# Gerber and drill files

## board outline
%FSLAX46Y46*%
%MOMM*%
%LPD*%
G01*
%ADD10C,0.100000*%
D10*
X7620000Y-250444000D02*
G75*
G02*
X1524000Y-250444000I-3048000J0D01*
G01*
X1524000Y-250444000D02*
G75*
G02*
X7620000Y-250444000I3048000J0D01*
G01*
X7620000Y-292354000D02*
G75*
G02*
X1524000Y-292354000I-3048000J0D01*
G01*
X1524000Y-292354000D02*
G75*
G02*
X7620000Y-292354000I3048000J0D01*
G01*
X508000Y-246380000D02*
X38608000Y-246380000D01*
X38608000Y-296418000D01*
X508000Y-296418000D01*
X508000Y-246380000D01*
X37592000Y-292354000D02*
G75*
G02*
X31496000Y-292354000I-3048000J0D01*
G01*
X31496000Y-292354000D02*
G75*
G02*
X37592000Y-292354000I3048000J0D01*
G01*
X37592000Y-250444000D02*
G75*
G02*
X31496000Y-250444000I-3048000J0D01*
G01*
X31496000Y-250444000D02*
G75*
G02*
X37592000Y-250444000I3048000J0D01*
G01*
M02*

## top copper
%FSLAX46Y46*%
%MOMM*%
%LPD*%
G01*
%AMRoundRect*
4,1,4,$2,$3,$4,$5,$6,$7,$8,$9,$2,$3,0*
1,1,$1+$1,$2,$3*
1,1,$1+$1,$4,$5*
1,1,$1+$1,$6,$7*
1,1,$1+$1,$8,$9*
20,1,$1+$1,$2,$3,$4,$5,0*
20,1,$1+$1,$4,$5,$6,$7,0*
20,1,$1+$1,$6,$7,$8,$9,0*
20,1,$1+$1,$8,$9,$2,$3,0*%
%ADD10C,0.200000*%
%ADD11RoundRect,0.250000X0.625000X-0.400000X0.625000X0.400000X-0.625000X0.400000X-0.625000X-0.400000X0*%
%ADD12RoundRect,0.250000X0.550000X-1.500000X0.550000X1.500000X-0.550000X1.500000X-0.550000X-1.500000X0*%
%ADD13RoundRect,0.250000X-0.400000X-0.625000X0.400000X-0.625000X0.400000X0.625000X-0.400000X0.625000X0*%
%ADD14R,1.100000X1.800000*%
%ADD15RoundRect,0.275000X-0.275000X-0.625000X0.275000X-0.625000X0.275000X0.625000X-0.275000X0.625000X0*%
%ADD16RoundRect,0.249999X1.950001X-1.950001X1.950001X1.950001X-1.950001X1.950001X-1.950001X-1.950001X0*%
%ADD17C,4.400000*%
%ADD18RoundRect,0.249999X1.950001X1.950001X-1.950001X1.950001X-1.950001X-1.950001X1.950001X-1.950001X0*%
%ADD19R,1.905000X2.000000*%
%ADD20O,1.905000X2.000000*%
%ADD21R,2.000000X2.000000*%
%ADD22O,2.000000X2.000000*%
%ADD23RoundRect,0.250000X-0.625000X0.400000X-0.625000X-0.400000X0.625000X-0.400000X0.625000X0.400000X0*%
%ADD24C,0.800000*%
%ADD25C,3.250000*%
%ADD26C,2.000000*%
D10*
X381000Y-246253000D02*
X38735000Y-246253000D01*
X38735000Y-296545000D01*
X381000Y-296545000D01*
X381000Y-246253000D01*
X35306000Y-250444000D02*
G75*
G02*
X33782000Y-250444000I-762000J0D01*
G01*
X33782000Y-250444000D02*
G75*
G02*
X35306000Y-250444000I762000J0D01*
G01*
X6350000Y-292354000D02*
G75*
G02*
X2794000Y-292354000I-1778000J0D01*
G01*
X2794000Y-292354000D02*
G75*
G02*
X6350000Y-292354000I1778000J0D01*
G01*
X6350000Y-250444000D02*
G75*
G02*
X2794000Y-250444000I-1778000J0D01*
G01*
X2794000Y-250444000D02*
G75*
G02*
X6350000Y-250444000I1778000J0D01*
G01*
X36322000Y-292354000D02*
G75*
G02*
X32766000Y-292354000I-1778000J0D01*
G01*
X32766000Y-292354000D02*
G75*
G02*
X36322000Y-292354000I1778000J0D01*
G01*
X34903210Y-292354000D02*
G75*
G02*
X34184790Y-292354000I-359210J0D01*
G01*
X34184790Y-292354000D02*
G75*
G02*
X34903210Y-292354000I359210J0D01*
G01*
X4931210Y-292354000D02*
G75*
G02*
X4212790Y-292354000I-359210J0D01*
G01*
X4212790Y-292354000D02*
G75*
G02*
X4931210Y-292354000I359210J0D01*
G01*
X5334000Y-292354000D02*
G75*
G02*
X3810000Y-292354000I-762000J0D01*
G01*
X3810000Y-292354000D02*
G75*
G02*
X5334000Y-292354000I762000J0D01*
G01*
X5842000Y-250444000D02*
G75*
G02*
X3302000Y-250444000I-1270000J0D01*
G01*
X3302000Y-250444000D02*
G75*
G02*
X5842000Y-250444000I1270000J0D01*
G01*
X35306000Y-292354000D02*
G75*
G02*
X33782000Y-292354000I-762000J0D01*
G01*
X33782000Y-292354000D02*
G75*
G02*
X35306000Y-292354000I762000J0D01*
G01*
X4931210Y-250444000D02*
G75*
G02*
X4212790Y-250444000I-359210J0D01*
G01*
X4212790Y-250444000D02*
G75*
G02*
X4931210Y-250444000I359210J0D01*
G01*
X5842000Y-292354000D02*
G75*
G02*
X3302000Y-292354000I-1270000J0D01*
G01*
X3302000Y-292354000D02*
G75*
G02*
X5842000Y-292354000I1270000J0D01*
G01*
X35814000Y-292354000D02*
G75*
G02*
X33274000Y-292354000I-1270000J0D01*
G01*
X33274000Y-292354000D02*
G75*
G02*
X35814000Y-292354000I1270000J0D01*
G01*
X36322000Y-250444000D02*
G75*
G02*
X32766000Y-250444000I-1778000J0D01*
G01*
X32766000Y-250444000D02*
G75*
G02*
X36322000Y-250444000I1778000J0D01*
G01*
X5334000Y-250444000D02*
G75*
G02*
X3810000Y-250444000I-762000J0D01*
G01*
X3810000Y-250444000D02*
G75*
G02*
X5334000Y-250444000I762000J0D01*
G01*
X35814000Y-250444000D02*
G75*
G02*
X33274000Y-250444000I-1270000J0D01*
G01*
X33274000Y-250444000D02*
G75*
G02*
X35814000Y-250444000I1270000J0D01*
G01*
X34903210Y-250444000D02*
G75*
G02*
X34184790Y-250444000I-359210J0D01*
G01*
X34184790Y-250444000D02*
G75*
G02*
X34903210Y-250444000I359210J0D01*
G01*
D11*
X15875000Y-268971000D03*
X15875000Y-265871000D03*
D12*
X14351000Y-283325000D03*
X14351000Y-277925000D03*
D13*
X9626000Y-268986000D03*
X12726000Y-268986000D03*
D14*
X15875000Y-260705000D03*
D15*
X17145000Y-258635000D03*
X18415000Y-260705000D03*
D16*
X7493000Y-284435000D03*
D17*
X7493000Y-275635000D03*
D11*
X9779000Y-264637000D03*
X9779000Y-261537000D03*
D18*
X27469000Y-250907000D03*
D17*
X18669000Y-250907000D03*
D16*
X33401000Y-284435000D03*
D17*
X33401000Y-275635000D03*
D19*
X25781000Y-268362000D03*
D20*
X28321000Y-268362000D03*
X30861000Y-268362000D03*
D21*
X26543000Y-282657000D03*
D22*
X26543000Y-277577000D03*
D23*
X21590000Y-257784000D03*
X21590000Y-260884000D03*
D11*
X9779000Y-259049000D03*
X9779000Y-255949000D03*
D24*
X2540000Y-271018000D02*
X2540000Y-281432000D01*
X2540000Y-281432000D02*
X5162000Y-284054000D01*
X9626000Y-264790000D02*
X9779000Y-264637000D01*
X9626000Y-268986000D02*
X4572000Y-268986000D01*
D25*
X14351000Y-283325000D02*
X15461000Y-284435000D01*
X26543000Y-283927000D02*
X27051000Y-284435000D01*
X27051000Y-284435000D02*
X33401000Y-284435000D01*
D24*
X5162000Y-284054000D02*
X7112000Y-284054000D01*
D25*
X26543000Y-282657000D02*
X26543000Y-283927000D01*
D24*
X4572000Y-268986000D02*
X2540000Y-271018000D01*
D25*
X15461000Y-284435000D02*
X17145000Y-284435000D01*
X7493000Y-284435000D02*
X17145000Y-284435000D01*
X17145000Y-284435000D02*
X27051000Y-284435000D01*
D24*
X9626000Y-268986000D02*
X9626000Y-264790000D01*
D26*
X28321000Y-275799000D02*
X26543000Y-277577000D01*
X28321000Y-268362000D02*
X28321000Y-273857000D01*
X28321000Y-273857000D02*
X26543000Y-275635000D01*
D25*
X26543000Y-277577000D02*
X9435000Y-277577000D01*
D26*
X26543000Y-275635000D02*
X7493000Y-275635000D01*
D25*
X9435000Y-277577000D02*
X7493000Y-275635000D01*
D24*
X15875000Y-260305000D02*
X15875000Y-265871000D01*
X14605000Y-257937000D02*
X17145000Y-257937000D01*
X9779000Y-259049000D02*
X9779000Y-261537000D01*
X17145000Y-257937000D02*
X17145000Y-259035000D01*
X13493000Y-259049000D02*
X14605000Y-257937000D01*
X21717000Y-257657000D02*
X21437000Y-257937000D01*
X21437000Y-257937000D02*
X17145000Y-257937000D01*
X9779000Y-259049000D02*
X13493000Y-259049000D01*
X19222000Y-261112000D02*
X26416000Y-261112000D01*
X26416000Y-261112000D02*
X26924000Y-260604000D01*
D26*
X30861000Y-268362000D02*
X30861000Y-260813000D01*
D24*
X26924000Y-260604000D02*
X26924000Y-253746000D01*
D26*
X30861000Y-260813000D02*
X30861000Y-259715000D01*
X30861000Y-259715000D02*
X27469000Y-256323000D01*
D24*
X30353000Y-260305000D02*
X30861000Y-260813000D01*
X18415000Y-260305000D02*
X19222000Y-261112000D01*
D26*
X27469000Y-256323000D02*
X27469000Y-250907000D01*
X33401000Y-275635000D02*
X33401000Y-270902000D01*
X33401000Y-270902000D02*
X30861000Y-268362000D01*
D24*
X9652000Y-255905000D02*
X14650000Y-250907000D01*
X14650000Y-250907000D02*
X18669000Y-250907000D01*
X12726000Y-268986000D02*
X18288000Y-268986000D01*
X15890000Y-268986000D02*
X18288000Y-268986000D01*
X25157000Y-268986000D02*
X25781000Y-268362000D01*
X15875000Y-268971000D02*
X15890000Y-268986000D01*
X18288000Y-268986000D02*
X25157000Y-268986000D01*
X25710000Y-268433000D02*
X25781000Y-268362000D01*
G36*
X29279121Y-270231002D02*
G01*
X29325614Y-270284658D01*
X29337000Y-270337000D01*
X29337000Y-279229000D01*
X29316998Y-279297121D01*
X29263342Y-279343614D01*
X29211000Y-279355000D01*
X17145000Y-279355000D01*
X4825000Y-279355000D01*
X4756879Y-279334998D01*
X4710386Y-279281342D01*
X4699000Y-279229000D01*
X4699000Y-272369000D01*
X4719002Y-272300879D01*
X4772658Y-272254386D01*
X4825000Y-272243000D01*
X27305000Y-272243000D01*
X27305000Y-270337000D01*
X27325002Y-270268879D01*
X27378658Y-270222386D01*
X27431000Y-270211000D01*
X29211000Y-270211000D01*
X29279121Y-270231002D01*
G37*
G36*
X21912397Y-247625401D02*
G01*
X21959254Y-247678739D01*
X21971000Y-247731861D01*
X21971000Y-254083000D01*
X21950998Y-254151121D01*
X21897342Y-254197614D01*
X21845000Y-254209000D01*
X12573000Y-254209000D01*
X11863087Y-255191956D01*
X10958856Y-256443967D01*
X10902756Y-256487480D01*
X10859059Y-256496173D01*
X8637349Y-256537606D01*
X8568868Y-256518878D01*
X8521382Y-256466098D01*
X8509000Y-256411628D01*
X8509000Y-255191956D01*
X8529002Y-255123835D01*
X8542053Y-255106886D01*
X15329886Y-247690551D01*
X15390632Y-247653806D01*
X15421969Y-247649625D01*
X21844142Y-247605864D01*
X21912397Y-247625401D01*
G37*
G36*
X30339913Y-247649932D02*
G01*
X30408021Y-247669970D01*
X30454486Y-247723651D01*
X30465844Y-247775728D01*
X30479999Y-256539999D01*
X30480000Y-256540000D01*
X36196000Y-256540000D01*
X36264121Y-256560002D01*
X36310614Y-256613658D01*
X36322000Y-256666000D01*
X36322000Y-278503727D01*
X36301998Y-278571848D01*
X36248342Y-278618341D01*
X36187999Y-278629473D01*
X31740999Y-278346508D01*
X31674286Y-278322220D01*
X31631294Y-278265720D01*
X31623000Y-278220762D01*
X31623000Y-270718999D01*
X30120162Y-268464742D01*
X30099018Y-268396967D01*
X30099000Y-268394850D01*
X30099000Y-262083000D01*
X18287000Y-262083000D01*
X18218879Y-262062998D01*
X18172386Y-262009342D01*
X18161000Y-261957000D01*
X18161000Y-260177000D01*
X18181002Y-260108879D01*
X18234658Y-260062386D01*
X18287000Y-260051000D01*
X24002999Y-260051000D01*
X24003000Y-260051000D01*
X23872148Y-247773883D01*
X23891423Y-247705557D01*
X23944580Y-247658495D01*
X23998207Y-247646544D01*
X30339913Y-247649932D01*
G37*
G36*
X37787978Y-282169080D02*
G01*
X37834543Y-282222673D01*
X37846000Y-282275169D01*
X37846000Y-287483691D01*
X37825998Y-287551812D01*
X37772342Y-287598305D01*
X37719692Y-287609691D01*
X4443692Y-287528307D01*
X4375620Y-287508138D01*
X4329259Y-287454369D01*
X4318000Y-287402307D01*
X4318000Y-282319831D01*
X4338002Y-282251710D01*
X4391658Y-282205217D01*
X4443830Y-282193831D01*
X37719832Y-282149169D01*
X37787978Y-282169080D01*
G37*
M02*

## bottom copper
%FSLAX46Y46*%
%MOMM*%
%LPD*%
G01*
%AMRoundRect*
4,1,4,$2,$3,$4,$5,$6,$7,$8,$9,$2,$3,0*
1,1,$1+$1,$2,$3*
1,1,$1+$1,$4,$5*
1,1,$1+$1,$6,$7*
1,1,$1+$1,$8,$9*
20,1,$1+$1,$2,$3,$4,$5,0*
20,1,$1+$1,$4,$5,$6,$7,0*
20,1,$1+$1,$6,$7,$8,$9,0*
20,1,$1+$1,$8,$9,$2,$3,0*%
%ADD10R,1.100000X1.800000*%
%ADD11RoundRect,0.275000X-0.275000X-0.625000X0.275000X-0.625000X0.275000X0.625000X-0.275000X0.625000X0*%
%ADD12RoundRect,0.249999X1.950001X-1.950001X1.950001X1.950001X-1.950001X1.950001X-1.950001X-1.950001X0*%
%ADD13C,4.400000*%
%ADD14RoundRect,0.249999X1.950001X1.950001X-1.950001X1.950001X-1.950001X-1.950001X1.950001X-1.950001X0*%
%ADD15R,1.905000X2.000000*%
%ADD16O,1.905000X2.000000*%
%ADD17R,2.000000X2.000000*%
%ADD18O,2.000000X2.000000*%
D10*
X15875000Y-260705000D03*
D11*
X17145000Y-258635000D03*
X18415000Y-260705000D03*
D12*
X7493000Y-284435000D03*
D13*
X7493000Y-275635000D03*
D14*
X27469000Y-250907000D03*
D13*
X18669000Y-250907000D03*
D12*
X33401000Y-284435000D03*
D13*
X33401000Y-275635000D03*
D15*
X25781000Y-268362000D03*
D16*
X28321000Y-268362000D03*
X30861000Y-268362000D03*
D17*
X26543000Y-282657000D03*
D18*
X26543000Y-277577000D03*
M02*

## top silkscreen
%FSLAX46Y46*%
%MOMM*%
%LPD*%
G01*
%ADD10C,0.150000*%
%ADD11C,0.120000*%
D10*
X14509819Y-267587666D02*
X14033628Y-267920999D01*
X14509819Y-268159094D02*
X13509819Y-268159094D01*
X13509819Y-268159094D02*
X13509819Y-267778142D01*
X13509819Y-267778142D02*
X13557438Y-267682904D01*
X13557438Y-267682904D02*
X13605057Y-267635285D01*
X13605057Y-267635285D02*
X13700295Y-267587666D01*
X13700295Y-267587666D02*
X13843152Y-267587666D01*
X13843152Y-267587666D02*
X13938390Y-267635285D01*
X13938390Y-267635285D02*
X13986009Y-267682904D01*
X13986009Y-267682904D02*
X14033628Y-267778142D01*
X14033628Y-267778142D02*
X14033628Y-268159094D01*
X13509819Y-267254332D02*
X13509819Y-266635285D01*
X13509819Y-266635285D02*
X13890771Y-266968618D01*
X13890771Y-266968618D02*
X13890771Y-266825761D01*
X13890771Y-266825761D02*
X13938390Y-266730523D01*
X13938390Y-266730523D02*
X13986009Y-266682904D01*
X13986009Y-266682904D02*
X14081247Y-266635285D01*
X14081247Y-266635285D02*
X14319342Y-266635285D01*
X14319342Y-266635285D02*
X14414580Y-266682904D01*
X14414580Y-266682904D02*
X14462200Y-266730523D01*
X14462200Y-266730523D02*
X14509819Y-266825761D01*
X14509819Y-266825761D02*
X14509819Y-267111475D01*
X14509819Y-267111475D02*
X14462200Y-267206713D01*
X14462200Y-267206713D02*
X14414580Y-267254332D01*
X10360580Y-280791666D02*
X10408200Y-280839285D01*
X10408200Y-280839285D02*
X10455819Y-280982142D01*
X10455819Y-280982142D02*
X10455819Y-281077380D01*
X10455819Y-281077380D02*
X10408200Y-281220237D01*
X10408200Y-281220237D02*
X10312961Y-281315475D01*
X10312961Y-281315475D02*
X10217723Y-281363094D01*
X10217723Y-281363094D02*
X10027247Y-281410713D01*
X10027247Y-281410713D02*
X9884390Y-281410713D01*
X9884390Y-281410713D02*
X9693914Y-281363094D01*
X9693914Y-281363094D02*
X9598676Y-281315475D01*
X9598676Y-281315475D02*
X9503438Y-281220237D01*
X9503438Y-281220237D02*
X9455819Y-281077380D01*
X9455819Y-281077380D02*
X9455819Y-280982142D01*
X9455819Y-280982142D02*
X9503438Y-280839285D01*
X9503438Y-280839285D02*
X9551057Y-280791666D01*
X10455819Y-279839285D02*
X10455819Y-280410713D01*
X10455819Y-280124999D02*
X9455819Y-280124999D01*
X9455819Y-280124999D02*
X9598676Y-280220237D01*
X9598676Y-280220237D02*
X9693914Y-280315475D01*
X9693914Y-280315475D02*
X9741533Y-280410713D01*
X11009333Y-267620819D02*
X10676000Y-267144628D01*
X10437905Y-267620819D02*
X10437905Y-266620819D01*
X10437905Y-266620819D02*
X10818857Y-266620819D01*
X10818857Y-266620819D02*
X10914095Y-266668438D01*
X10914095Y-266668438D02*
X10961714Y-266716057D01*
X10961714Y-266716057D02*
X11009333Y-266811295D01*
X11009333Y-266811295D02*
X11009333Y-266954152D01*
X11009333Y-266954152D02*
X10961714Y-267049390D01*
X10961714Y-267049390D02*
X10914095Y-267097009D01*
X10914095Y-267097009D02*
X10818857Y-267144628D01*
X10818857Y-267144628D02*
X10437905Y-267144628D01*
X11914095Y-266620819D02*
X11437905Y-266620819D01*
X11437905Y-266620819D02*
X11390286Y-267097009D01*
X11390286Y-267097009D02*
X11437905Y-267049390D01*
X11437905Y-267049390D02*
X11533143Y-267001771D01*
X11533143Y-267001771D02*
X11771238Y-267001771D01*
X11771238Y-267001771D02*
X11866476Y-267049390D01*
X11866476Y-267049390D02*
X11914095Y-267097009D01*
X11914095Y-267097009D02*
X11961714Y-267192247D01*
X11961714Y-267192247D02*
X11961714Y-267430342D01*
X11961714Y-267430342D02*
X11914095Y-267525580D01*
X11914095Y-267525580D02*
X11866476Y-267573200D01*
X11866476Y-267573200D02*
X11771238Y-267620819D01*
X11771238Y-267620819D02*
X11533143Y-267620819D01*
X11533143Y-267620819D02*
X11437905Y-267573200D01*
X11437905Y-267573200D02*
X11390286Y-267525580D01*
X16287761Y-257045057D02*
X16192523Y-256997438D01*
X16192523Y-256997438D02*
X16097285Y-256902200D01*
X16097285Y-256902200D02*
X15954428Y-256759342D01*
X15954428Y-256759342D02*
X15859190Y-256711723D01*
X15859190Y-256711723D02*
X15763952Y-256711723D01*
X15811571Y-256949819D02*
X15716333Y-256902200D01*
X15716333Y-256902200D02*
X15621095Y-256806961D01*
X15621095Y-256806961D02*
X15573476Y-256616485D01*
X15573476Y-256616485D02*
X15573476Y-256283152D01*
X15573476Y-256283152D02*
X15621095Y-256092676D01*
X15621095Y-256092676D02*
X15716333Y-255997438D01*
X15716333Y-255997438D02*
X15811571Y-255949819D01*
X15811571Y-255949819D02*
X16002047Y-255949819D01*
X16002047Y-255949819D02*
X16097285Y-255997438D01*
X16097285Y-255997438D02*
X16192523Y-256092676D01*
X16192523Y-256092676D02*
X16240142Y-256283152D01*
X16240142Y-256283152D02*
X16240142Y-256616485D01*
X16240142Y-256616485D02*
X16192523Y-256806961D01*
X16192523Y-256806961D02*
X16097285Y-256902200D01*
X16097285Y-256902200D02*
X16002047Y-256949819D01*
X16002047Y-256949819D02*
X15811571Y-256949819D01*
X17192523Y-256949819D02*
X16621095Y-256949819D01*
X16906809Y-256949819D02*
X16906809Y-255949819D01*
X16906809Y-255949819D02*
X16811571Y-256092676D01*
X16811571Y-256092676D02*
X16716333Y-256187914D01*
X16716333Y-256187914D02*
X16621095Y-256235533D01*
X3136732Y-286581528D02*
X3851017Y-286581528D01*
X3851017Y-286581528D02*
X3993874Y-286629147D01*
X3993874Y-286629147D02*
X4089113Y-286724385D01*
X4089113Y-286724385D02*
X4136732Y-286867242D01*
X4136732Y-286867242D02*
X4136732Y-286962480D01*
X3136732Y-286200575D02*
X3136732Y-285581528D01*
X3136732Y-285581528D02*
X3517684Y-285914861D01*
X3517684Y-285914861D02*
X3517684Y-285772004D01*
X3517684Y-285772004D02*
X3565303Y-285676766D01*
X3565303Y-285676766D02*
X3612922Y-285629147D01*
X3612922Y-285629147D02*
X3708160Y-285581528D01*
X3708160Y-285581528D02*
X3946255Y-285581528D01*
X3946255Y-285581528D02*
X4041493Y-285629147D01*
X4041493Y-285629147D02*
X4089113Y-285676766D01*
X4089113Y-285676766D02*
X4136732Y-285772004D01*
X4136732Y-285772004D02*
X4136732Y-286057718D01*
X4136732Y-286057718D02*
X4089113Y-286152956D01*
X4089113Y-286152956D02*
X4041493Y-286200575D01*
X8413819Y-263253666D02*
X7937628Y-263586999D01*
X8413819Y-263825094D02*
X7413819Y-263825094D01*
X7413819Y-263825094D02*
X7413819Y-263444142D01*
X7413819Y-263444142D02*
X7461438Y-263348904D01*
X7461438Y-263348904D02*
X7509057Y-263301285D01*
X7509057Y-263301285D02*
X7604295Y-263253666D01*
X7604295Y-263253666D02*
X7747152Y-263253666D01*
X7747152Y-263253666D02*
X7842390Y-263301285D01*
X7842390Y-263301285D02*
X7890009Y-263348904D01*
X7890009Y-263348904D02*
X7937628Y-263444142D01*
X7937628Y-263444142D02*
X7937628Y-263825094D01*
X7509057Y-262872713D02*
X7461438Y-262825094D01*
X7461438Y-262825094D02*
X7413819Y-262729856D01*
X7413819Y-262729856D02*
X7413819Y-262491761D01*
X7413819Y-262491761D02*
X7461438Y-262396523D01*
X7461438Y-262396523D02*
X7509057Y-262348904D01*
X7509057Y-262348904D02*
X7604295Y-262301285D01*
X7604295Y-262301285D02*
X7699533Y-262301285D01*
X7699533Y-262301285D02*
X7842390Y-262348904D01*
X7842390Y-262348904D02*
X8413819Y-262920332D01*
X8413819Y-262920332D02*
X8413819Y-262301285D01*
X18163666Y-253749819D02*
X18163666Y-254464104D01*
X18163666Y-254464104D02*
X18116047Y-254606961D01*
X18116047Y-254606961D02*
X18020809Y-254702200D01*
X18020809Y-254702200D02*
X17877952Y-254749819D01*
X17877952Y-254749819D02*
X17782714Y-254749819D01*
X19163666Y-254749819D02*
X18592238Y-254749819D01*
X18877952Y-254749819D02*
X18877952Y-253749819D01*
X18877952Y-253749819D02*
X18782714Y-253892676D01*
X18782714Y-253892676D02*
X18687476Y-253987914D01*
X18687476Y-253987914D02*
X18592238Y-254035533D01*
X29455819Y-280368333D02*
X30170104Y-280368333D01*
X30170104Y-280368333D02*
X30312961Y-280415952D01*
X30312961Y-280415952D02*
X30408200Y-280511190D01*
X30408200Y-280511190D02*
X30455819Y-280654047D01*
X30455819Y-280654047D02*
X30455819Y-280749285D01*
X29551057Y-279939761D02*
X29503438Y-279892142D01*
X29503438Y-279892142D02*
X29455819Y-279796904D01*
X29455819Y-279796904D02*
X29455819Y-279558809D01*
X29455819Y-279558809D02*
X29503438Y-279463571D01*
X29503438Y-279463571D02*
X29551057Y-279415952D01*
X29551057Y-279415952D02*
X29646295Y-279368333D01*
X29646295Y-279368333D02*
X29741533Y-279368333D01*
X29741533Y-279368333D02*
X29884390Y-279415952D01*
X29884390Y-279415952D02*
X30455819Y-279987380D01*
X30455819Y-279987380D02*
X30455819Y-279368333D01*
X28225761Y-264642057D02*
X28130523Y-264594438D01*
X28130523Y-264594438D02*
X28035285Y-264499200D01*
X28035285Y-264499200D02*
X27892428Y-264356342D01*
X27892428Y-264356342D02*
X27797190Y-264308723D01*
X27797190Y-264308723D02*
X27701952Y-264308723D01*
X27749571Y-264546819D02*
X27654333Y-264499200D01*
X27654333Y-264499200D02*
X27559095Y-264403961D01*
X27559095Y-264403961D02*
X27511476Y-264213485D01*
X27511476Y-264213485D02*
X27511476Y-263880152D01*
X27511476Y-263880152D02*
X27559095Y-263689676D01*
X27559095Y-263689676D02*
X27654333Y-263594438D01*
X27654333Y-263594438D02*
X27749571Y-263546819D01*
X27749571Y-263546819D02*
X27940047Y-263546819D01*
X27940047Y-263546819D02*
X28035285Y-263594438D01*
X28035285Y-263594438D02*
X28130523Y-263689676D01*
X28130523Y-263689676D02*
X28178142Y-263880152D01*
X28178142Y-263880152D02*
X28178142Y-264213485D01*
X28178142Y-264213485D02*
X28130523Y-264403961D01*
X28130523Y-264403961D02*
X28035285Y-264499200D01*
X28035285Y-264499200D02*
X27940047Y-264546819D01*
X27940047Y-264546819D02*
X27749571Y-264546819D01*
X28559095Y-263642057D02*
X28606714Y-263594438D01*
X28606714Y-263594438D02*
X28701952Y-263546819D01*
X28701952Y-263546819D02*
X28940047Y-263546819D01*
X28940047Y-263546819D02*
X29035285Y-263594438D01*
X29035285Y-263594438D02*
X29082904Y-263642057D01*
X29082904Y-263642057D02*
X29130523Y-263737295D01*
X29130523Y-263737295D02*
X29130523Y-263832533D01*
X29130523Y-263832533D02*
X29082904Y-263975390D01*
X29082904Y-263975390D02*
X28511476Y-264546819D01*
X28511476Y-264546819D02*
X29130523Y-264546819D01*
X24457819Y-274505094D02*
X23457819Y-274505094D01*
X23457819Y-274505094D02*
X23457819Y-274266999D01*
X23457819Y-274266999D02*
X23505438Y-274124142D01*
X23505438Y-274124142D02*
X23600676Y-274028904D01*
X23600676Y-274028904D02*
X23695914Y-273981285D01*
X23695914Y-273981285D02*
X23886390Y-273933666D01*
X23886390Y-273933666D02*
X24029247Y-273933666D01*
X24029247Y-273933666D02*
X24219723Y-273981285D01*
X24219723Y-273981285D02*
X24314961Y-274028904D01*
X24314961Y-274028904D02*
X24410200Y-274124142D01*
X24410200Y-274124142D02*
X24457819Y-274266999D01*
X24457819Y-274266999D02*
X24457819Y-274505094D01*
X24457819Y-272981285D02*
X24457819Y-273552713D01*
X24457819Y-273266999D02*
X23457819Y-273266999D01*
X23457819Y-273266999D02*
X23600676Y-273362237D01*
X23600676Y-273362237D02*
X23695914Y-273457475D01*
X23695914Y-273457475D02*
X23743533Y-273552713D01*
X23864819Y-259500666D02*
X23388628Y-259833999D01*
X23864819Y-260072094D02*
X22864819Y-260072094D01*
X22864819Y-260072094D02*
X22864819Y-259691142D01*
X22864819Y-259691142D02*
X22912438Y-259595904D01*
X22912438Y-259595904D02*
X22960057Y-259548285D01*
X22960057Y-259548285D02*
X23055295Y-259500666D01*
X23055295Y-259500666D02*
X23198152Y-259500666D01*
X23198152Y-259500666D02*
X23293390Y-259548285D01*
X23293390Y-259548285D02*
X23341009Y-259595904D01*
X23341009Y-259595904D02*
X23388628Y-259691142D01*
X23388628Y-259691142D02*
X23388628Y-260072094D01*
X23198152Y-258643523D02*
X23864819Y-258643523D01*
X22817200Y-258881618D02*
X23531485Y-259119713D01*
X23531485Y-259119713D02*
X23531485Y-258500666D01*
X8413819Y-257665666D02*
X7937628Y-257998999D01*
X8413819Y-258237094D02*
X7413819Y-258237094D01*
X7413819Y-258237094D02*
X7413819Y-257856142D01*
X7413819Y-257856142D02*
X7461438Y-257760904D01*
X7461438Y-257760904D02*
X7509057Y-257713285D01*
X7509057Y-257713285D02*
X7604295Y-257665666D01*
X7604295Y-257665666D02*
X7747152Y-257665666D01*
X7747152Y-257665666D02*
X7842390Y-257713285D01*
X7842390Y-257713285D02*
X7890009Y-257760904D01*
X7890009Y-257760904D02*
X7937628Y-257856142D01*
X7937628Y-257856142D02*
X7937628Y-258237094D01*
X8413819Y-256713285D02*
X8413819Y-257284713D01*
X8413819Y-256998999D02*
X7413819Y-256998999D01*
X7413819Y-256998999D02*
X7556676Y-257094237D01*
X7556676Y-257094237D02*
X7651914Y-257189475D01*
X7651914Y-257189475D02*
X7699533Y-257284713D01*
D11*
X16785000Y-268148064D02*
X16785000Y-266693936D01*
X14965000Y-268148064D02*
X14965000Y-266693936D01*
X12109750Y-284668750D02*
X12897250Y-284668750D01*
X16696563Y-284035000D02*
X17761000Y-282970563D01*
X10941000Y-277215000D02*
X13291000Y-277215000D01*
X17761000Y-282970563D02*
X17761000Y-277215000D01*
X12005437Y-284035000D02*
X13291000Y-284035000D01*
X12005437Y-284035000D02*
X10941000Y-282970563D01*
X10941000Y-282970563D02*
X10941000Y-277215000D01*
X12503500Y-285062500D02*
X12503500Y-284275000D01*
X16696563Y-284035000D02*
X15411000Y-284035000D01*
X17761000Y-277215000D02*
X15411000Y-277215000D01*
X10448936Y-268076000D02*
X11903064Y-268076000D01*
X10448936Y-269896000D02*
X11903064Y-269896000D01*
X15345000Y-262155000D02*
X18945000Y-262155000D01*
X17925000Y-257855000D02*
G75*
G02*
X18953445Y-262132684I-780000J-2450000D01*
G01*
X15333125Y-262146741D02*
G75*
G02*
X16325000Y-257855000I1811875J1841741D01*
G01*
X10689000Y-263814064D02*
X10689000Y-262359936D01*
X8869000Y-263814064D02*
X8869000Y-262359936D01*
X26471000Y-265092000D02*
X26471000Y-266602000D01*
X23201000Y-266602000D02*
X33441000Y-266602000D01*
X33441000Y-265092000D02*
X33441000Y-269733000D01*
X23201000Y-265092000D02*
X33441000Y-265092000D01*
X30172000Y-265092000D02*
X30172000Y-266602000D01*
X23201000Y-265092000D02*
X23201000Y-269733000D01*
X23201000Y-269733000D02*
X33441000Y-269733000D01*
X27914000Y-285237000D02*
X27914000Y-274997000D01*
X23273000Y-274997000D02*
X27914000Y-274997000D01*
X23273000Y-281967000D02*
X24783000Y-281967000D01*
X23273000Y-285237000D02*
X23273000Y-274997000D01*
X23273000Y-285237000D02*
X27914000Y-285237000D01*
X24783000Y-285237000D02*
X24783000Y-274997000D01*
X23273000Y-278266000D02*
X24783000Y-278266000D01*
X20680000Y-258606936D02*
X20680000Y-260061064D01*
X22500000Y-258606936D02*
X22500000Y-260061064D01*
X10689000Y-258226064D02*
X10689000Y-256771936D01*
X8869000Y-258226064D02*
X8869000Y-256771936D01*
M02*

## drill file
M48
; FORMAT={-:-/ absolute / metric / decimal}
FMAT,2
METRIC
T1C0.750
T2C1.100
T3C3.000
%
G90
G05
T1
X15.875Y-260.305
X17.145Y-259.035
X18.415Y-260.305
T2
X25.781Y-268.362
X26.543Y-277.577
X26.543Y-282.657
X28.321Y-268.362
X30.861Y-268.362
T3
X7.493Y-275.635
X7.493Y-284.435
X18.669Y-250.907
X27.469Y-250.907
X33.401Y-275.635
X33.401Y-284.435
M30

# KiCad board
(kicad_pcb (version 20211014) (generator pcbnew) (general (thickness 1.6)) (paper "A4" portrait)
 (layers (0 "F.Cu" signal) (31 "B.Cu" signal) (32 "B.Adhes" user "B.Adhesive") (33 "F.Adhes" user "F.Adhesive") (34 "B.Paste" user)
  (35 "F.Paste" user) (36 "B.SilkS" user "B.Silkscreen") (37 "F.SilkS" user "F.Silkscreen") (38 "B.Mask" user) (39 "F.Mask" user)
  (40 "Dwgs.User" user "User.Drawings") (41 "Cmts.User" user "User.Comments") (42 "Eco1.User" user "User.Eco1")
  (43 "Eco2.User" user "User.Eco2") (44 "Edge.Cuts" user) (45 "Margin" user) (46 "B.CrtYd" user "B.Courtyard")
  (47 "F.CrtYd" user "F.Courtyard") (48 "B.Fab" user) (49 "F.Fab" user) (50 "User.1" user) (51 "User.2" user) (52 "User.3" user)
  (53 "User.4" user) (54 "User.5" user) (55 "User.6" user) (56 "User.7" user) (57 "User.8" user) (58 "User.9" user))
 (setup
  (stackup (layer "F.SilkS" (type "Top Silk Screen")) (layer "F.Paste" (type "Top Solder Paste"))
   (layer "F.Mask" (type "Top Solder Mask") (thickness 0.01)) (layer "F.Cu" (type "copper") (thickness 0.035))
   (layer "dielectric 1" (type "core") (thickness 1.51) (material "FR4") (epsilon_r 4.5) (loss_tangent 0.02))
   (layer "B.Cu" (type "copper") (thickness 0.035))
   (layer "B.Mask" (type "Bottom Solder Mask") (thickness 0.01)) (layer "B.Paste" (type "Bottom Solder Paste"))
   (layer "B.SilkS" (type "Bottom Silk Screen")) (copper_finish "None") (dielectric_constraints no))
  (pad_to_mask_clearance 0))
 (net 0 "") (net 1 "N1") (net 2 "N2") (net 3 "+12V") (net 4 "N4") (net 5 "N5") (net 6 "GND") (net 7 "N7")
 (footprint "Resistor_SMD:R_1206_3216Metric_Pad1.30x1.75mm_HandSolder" (layer "F.Cu") (at 15.875 267.421 90)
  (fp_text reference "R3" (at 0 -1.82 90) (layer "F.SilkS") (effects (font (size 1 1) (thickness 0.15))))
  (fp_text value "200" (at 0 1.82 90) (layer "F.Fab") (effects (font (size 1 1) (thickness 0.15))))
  (fp_line (start -0.727064 0.91) (end 0.727064 0.91) (layer "F.SilkS") (width 0.12))
  (fp_line (start -0.727064 -0.91) (end 0.727064 -0.91) (layer "F.SilkS") (width 0.12))
  (pad "1" smd roundrect (at -1.55 0 90) (size 1.3 1.75) (layers "F.Cu" "F.Paste" "F.Mask") (roundrect_rratio 0.192308) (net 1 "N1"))
  (pad "2" smd roundrect (at 1.55 0 90) (size 1.3 1.75) (layers "F.Cu" "F.Paste" "F.Mask") (roundrect_rratio 0.192308) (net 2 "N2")))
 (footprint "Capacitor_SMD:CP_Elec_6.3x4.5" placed (layer "F.Cu") (at 14.351 280.625 90)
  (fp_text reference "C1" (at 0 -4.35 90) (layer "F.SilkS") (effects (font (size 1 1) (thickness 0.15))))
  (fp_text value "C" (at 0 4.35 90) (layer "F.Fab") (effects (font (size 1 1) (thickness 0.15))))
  (fp_line (start -4.04375 -2.24125) (end -4.04375 -1.45375) (layer "F.SilkS") (width 0.12))
  (fp_line (start -3.41 2.345563) (end -2.345563 3.41) (layer "F.SilkS") (width 0.12))
  (fp_line (start 3.41 -3.41) (end 3.41 -1.06) (layer "F.SilkS") (width 0.12))
  (fp_line (start -2.345563 3.41) (end 3.41 3.41) (layer "F.SilkS") (width 0.12))
  (fp_line (start -3.41 -2.345563) (end -3.41 -1.06) (layer "F.SilkS") (width 0.12))
  (fp_line (start -3.41 -2.345563) (end -2.345563 -3.41) (layer "F.SilkS") (width 0.12))
  (fp_line (start -2.345563 -3.41) (end 3.41 -3.41) (layer "F.SilkS") (width 0.12))
  (fp_line (start -4.4375 -1.8475) (end -3.65 -1.8475) (layer "F.SilkS") (width 0.12))
  (fp_line (start -3.41 2.345563) (end -3.41 1.06) (layer "F.SilkS") (width 0.12))
  (fp_line (start 3.41 3.41) (end 3.41 1.06) (layer "F.SilkS") (width 0.12))
  (pad "1" smd roundrect (at -2.7 0 90) (size 3.5 1.6) (layers "F.Cu" "F.Paste" "F.Mask") (roundrect_rratio 0.15625) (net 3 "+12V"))
  (pad "2" smd roundrect (at 2.7 0 90) (size 3.5 1.6) (layers "F.Cu" "F.Paste" "F.Mask") (roundrect_rratio 0.15625) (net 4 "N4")))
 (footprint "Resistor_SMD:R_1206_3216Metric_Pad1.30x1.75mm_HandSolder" (layer "F.Cu") (at 11.176 268.986)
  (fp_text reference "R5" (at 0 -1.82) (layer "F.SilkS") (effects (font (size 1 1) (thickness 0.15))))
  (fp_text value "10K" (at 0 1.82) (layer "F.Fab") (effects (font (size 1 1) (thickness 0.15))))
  (fp_line (start -0.727064 -0.91) (end 0.727064 -0.91) (layer "F.SilkS") (width 0.12))
  (fp_line (start -0.727064 0.91) (end 0.727064 0.91) (layer "F.SilkS") (width 0.12))
  (pad "1" smd roundrect (at -1.55 0) (size 1.3 1.75) (layers "F.Cu" "F.Paste" "F.Mask") (roundrect_rratio 0.192308) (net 3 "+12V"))
  (pad "2" smd roundrect (at 1.55 0) (size 1.3 1.75) (layers "F.Cu" "F.Paste" "F.Mask") (roundrect_rratio 0.192308) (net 1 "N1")))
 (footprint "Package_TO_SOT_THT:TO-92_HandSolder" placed (layer "F.Cu") (at 15.875 260.305)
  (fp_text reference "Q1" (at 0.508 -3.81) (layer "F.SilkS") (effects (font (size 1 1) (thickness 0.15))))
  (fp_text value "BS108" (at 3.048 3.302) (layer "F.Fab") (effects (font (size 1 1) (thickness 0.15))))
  (fp_line (start -0.53 1.85) (end 3.07 1.85) (layer "F.SilkS") (width 0.12))
  (fp_arc (start 2.05 -2.45) (mid 3.769931 -0.601036) (end 3.078445 1.827684) (layer "F.SilkS") (width 0.12))
  (fp_arc (start -0.541875 1.841741) (mid -1.247231 -0.581764) (end 0.45 -2.45) (layer "F.SilkS") (width 0.12))
  (pad "1" thru_hole rect (at 0 0) (size 1.1 1.8) (drill 0.75 (offset 0 0.4)) (layers *.Cu *.Mask) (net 2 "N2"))
  (pad "2" thru_hole roundrect (at 1.27 -1.27) (size 1.1 1.8) (drill 0.75 (offset 0 -0.4)) (layers *.Cu *.Mask) (roundrect_rratio 0.25)
   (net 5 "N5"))
  (pad "3" thru_hole roundrect (at 2.54 0) (size 1.1 1.8) (drill 0.75 (offset 0 0.4)) (layers *.Cu *.Mask) (roundrect_rratio 0.25)
   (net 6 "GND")))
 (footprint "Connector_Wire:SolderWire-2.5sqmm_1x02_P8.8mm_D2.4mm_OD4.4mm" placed (layer "F.Cu") (at 7.493 284.435 90)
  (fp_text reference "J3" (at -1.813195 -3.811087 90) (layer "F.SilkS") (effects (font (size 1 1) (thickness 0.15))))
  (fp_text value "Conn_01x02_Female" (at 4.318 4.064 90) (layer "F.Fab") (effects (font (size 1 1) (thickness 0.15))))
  (pad "1" thru_hole roundrect (at 0 0 90) (size 4.4 4.4) (drill 3) (layers *.Cu *.Mask) (roundrect_rratio 0.05681795455) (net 3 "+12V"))
  (pad "2" thru_hole circle (at 8.8 0 90) (size 4.4 4.4) (drill 3) (layers *.Cu *.Mask) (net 4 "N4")))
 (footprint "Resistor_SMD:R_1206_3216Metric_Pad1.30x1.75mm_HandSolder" (layer "F.Cu") (at 9.779 263.087 90)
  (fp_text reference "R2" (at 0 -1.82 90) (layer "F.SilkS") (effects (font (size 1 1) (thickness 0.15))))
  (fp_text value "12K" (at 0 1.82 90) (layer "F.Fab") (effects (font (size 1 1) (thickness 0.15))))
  (fp_line (start -0.727064 0.91) (end 0.727064 0.91) (layer "F.SilkS") (width 0.12))
  (fp_line (start -0.727064 -0.91) (end 0.727064 -0.91) (layer "F.SilkS") (width 0.12))
  (pad "1" smd roundrect (at -1.55 0 90) (size 1.3 1.75) (layers "F.Cu" "F.Paste" "F.Mask") (roundrect_rratio 0.192308) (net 3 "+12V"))
  (pad "2" smd roundrect (at 1.55 0 90) (size 1.3 1.75) (layers "F.Cu" "F.Paste" "F.Mask") (roundrect_rratio 0.192308) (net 5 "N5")))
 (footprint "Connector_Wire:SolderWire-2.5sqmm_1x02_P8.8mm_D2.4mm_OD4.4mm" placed (layer "F.Cu") (at 27.469 250.907 180)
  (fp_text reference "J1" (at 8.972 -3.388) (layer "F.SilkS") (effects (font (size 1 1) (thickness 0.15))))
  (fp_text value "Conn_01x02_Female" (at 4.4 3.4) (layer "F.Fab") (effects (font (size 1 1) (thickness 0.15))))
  (pad "1" thru_hole roundrect (at 0 0 180) (size 4.4 4.4) (drill 3) (layers *.Cu *.Mask) (roundrect_rratio 0.05681795455) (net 6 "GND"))
  (pad "2" thru_hole circle (at 8.8 0 180) (size 4.4 4.4) (drill 3) (layers *.Cu *.Mask) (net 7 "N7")))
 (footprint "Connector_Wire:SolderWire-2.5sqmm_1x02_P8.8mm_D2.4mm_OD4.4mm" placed (layer "F.Cu") (at 33.401 284.435 90)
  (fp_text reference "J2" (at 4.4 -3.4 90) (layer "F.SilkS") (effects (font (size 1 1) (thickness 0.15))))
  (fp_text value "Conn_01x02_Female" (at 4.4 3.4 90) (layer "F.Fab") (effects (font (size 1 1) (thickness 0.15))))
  (pad "1" thru_hole roundrect (at 0 0 90) (size 4.4 4.4) (drill 3) (layers *.Cu *.Mask) (roundrect_rratio 0.05681795455) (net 3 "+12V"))
  (pad "2" thru_hole circle (at 8.8 0 90) (size 4.4 4.4) (drill 3) (layers *.Cu *.Mask) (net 6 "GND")))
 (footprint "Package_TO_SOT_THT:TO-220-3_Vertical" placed (layer "F.Cu") (at 25.781 268.362)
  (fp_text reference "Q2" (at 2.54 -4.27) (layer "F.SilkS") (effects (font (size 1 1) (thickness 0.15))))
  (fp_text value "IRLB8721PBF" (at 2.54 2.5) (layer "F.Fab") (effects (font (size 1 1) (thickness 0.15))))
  (fp_line (start 0.69 -3.27) (end 0.69 -1.76) (layer "F.SilkS") (width 0.12))
  (fp_line (start -2.58 -1.76) (end 7.66 -1.76) (layer "F.SilkS") (width 0.12))
  (fp_line (start 7.66 -3.27) (end 7.66 1.371) (layer "F.SilkS") (width 0.12))
  (fp_line (start -2.58 -3.27) (end 7.66 -3.27) (layer "F.SilkS") (width 0.12))
  (fp_line (start 4.391 -3.27) (end 4.391 -1.76) (layer "F.SilkS") (width 0.12))
  (fp_line (start -2.58 -3.27) (end -2.58 1.371) (layer "F.SilkS") (width 0.12))
  (fp_line (start -2.58 1.371) (end 7.66 1.371) (layer "F.SilkS") (width 0.12))
  (pad "1" thru_hole rect (at 0 0) (size 1.905 2) (drill 1.1) (layers *.Cu *.Mask) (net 1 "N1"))
  (pad "2" thru_hole oval (at 2.54 0) (size 1.905 2) (drill 1.1) (layers *.Cu *.Mask) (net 4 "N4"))
  (pad "3" thru_hole oval (at 5.08 0) (size 1.905 2) (drill 1.1) (layers *.Cu *.Mask) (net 6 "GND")))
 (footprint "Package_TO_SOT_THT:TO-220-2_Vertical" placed (layer "F.Cu") (at 26.543 282.657 90)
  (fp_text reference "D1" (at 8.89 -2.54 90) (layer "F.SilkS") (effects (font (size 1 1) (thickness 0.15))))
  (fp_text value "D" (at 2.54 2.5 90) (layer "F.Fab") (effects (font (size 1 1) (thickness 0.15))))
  (fp_line (start -2.58 1.371) (end 7.66 1.371) (layer "F.SilkS") (width 0.12))
  (fp_line (start 7.66 -3.27) (end 7.66 1.371) (layer "F.SilkS") (width 0.12))
  (fp_line (start 0.69 -3.27) (end 0.69 -1.76) (layer "F.SilkS") (width 0.12))
  (fp_line (start -2.58 -3.27) (end 7.66 -3.27) (layer "F.SilkS") (width 0.12))
  (fp_line (start -2.58 -3.27) (end -2.58 1.371) (layer "F.SilkS") (width 0.12))
  (fp_line (start -2.58 -1.76) (end 7.66 -1.76) (layer "F.SilkS") (width 0.12))
  (fp_line (start 4.391 -3.27) (end 4.391 -1.76) (layer "F.SilkS") (width 0.12))
  (pad "1" thru_hole rect (at 0 0 90) (size 2 2) (drill 1.1) (layers *.Cu *.Mask) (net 3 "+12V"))
  (pad "2" thru_hole oval (at 5.08 0 90) (size 2 2) (drill 1.1) (layers *.Cu *.Mask) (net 4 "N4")))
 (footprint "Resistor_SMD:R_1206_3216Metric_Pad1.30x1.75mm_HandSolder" (layer "F.Cu") (at 21.59 259.334 -90)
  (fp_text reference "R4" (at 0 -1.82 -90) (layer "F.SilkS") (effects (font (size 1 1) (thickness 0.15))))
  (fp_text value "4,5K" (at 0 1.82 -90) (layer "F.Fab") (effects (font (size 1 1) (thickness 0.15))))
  (fp_line (start -0.727064 0.91) (end 0.727064 0.91) (layer "F.SilkS") (width 0.12))
  (fp_line (start -0.727064 -0.91) (end 0.727064 -0.91) (layer "F.SilkS") (width 0.12))
  (pad "1" smd roundrect (at -1.55 0 270) (size 1.3 1.75) (layers "F.Cu" "F.Paste" "F.Mask") (roundrect_rratio 0.192308) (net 5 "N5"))
  (pad "2" smd roundrect (at 1.55 0 270) (size 1.3 1.75) (layers "F.Cu" "F.Paste" "F.Mask") (roundrect_rratio 0.192308) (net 6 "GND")))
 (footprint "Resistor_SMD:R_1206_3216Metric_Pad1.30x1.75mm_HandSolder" (layer "F.Cu") (at 9.779 257.499 90)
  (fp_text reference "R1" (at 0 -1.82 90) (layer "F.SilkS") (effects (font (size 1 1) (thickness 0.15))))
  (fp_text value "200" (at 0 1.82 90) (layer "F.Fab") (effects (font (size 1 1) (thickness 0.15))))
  (fp_line (start -0.727064 0.91) (end 0.727064 0.91) (layer "F.SilkS") (width 0.12))
  (fp_line (start -0.727064 -0.91) (end 0.727064 -0.91) (layer "F.SilkS") (width 0.12))
  (pad "1" smd roundrect (at -1.55 0 90) (size 1.3 1.75) (layers "F.Cu" "F.Paste" "F.Mask") (roundrect_rratio 0.192308) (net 5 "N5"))
  (pad "2" smd roundrect (at 1.55 0 90) (size 1.3 1.75) (layers "F.Cu" "F.Paste" "F.Mask") (roundrect_rratio 0.192308) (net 7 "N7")))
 (gr_rect (start 38.735 246.253) (end 0.381 296.545) (layer "F.Cu") (width 0.2) (fill none))
 (gr_circle (center 34.544 250.444) (end 35.306 250.444) (layer "F.Cu") (width 0.2) (fill none))
 (gr_circle (center 4.572 292.354) (end 6.35 292.354) (layer "F.Cu") (width 0.2) (fill none))
 (gr_circle (center 4.572 250.444) (end 6.35 250.444) (layer "F.Cu") (width 0.2) (fill none))
 (gr_circle (center 34.544 292.354) (end 36.322 292.354) (layer "F.Cu") (width 0.2) (fill none))
 (gr_circle (center 34.544 292.354) (end 34.90321 292.354) (layer "F.Cu") (width 0.2) (fill none))
 (gr_circle (center 4.572 292.354) (end 4.93121 292.354) (layer "F.Cu") (width 0.2) (fill none))
 (gr_circle (center 4.572 292.354) (end 5.334 292.354) (layer "F.Cu") (width 0.2) (fill none))
 (gr_circle (center 4.572 250.444) (end 5.842 250.444) (layer "F.Cu") (width 0.2) (fill none))
 (gr_circle (center 34.544 292.354) (end 35.306 292.354) (layer "F.Cu") (width 0.2) (fill none))
 (gr_circle (center 4.572 250.444) (end 4.93121 250.444) (layer "F.Cu") (width 0.2) (fill none))
 (gr_circle (center 4.572 292.354) (end 5.842 292.354) (layer "F.Cu") (width 0.2) (fill none))
 (gr_circle (center 34.544 292.354) (end 35.814 292.354) (layer "F.Cu") (width 0.2) (fill none))
 (gr_circle (center 34.544 250.444) (end 36.322 250.444) (layer "F.Cu") (width 0.2) (fill none))
 (gr_circle (center 4.572 250.444) (end 5.334 250.444) (layer "F.Cu") (width 0.2) (fill none))
 (gr_circle (center 34.544 250.444) (end 35.814 250.444) (layer "F.Cu") (width 0.2) (fill none))
 (gr_circle (center 34.544 250.444) (end 34.90321 250.444) (layer "F.Cu") (width 0.2) (fill none))
 (gr_circle (center 4.572 250.444) (end 4.572 247.396) (layer "Edge.Cuts") (width 0.1) (fill none))
 (gr_circle (center 4.572 292.354) (end 1.524 292.354) (layer "Edge.Cuts") (width 0.1) (fill none))
 (gr_rect (start 0.508 246.38) (end 38.608 296.418) (layer "Edge.Cuts") (width 0.1) (fill none))
 (gr_circle (center 34.544 292.354) (end 34.544 295.402) (layer "Edge.Cuts") (width 0.1) (fill none))
 (gr_circle (center 34.544 250.444) (end 37.592 250.444) (layer "Edge.Cuts") (width 0.1) (fill none))
 (segment (start 2.54 271.018) (end 2.54 281.432) (width 0.8) (layer "F.Cu") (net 3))
 (segment (start 2.54 281.432) (end 5.162 284.054) (width 0.8) (layer "F.Cu") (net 3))
 (segment (start 9.626 264.79) (end 9.779 264.637) (width 0.8) (layer "F.Cu") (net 3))
 (segment (start 9.626 268.986) (end 4.572 268.986) (width 0.8) (layer "F.Cu") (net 3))
 (segment (start 14.351 283.325) (end 15.461 284.435) (width 3.25) (layer "F.Cu") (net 3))
 (segment (start 26.543 283.927) (end 27.051 284.435) (width 3.25) (layer "F.Cu") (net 3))
 (segment (start 27.051 284.435) (end 33.401 284.435) (width 3.25) (layer "F.Cu") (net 3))
 (segment (start 5.162 284.054) (end 7.112 284.054) (width 0.8) (layer "F.Cu") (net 3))
 (segment (start 26.543 282.657) (end 26.543 283.927) (width 3.25) (layer "F.Cu") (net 3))
 (segment (start 4.572 268.986) (end 2.54 271.018) (width 0.8) (layer "F.Cu") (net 3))
 (segment (start 15.461 284.435) (end 17.145 284.435) (width 3.25) (layer "F.Cu") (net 3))
 (segment (start 7.493 284.435) (end 17.145 284.435) (width 3.25) (layer "F.Cu") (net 3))
 (segment (start 17.145 284.435) (end 27.051 284.435) (width 3.25) (layer "F.Cu") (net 3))
 (segment (start 9.626 268.986) (end 9.626 264.79) (width 0.8) (layer "F.Cu") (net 3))
 (segment (start 28.321 275.799) (end 26.543 277.577) (width 2) (layer "F.Cu") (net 4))
 (segment (start 28.321 268.362) (end 28.321 273.857) (width 2) (layer "F.Cu") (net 4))
 (segment (start 28.321 273.857) (end 26.543 275.635) (width 2) (layer "F.Cu") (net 4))
 (segment (start 26.543 277.577) (end 9.435 277.577) (width 3.25) (layer "F.Cu") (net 4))
 (segment (start 26.543 275.635) (end 7.493 275.635) (width 2) (layer "F.Cu") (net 4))
 (segment (start 9.435 277.577) (end 7.493 275.635) (width 3.25) (layer "F.Cu") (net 4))
 (segment (start 15.875 260.305) (end 15.875 265.871) (width 0.8) (layer "F.Cu") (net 2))
 (segment (start 14.605 257.937) (end 17.145 257.937) (width 0.8) (layer "F.Cu") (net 5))
 (segment (start 9.779 259.049) (end 9.779 261.537) (width 0.8) (layer "F.Cu") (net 5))
 (segment (start 17.145 257.937) (end 17.145 259.035) (width 0.8) (layer "F.Cu") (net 5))
 (segment (start 13.493 259.049) (end 14.605 257.937) (width 0.8) (layer "F.Cu") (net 5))
 (segment (start 21.717 257.657) (end 21.437 257.937) (width 0.8) (layer "F.Cu") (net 5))
 (segment (start 21.437 257.937) (end 17.145 257.937) (width 0.8) (layer "F.Cu") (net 5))
 (segment (start 9.779 259.049) (end 13.493 259.049) (width 0.8) (layer "F.Cu") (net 5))
 (segment (start 19.222 261.112) (end 26.416 261.112) (width 0.8) (layer "F.Cu") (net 6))
 (segment (start 26.416 261.112) (end 26.924 260.604) (width 0.8) (layer "F.Cu") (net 6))
 (segment (start 30.861 268.362) (end 30.861 260.813) (width 2) (layer "F.Cu") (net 6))
 (segment (start 26.924 260.604) (end 26.924 253.746) (width 0.8) (layer "F.Cu") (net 6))
 (segment (start 30.861 260.813) (end 30.861 259.715) (width 2) (layer "F.Cu") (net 6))
 (segment (start 30.861 259.715) (end 27.469 256.323) (width 2) (layer "F.Cu") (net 6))
 (segment (start 30.353 260.305) (end 30.861 260.813) (width 0.8) (layer "F.Cu") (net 6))
 (segment (start 18.415 260.305) (end 19.222 261.112) (width 0.8) (layer "F.Cu") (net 6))
 (segment (start 27.469 256.323) (end 27.469 250.907) (width 2) (layer "F.Cu") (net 6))
 (segment (start 33.401 275.635) (end 33.401 270.902) (width 2) (layer "F.Cu") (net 6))
 (segment (start 33.401 270.902) (end 30.861 268.362) (width 2) (layer "F.Cu") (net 6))
 (segment (start 9.652 255.905) (end 14.65 250.907) (width 0.8) (layer "F.Cu") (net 7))
 (segment (start 14.65 250.907) (end 18.669 250.907) (width 0.8) (layer "F.Cu") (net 7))
 (segment (start 12.726 268.986) (end 18.288 268.986) (width 0.8) (layer "F.Cu") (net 1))
 (segment (start 15.89 268.986) (end 18.288 268.986) (width 0.8) (layer "F.Cu") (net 1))
 (segment (start 25.157 268.986) (end 25.781 268.362) (width 0.8) (layer "F.Cu") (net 1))
 (segment (start 15.875 268.971) (end 15.89 268.986) (width 0.8) (layer "F.Cu") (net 1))
 (segment (start 18.288 268.986) (end 25.157 268.986) (width 0.8) (layer "F.Cu") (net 1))
 (segment (start 25.71 268.433) (end 25.781 268.362) (width 0.8) (layer "F.Cu") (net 1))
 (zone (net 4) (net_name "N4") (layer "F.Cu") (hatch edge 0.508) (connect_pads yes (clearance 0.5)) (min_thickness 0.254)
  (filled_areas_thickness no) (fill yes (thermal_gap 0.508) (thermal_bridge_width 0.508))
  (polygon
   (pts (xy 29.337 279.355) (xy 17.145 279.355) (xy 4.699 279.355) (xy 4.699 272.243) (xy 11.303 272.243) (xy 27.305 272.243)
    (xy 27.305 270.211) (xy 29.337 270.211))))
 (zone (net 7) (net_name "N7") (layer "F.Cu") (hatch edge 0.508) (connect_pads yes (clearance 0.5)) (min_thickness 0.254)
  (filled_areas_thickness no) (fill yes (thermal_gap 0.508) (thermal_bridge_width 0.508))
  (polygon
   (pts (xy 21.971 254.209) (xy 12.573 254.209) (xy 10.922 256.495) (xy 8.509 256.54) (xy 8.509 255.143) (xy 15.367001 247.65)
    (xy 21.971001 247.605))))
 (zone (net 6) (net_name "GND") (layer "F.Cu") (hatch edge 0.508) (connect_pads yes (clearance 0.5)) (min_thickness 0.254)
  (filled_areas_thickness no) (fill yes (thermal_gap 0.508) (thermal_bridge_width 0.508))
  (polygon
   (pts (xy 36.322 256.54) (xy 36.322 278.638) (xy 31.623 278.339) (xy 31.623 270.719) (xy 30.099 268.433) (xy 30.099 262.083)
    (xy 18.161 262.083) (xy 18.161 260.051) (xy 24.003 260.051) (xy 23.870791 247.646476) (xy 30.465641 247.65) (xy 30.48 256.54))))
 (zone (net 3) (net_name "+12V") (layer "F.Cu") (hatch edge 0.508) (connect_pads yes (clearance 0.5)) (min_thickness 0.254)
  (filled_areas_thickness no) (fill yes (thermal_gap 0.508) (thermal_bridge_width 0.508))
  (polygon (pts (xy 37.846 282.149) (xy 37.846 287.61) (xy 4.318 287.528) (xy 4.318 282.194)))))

